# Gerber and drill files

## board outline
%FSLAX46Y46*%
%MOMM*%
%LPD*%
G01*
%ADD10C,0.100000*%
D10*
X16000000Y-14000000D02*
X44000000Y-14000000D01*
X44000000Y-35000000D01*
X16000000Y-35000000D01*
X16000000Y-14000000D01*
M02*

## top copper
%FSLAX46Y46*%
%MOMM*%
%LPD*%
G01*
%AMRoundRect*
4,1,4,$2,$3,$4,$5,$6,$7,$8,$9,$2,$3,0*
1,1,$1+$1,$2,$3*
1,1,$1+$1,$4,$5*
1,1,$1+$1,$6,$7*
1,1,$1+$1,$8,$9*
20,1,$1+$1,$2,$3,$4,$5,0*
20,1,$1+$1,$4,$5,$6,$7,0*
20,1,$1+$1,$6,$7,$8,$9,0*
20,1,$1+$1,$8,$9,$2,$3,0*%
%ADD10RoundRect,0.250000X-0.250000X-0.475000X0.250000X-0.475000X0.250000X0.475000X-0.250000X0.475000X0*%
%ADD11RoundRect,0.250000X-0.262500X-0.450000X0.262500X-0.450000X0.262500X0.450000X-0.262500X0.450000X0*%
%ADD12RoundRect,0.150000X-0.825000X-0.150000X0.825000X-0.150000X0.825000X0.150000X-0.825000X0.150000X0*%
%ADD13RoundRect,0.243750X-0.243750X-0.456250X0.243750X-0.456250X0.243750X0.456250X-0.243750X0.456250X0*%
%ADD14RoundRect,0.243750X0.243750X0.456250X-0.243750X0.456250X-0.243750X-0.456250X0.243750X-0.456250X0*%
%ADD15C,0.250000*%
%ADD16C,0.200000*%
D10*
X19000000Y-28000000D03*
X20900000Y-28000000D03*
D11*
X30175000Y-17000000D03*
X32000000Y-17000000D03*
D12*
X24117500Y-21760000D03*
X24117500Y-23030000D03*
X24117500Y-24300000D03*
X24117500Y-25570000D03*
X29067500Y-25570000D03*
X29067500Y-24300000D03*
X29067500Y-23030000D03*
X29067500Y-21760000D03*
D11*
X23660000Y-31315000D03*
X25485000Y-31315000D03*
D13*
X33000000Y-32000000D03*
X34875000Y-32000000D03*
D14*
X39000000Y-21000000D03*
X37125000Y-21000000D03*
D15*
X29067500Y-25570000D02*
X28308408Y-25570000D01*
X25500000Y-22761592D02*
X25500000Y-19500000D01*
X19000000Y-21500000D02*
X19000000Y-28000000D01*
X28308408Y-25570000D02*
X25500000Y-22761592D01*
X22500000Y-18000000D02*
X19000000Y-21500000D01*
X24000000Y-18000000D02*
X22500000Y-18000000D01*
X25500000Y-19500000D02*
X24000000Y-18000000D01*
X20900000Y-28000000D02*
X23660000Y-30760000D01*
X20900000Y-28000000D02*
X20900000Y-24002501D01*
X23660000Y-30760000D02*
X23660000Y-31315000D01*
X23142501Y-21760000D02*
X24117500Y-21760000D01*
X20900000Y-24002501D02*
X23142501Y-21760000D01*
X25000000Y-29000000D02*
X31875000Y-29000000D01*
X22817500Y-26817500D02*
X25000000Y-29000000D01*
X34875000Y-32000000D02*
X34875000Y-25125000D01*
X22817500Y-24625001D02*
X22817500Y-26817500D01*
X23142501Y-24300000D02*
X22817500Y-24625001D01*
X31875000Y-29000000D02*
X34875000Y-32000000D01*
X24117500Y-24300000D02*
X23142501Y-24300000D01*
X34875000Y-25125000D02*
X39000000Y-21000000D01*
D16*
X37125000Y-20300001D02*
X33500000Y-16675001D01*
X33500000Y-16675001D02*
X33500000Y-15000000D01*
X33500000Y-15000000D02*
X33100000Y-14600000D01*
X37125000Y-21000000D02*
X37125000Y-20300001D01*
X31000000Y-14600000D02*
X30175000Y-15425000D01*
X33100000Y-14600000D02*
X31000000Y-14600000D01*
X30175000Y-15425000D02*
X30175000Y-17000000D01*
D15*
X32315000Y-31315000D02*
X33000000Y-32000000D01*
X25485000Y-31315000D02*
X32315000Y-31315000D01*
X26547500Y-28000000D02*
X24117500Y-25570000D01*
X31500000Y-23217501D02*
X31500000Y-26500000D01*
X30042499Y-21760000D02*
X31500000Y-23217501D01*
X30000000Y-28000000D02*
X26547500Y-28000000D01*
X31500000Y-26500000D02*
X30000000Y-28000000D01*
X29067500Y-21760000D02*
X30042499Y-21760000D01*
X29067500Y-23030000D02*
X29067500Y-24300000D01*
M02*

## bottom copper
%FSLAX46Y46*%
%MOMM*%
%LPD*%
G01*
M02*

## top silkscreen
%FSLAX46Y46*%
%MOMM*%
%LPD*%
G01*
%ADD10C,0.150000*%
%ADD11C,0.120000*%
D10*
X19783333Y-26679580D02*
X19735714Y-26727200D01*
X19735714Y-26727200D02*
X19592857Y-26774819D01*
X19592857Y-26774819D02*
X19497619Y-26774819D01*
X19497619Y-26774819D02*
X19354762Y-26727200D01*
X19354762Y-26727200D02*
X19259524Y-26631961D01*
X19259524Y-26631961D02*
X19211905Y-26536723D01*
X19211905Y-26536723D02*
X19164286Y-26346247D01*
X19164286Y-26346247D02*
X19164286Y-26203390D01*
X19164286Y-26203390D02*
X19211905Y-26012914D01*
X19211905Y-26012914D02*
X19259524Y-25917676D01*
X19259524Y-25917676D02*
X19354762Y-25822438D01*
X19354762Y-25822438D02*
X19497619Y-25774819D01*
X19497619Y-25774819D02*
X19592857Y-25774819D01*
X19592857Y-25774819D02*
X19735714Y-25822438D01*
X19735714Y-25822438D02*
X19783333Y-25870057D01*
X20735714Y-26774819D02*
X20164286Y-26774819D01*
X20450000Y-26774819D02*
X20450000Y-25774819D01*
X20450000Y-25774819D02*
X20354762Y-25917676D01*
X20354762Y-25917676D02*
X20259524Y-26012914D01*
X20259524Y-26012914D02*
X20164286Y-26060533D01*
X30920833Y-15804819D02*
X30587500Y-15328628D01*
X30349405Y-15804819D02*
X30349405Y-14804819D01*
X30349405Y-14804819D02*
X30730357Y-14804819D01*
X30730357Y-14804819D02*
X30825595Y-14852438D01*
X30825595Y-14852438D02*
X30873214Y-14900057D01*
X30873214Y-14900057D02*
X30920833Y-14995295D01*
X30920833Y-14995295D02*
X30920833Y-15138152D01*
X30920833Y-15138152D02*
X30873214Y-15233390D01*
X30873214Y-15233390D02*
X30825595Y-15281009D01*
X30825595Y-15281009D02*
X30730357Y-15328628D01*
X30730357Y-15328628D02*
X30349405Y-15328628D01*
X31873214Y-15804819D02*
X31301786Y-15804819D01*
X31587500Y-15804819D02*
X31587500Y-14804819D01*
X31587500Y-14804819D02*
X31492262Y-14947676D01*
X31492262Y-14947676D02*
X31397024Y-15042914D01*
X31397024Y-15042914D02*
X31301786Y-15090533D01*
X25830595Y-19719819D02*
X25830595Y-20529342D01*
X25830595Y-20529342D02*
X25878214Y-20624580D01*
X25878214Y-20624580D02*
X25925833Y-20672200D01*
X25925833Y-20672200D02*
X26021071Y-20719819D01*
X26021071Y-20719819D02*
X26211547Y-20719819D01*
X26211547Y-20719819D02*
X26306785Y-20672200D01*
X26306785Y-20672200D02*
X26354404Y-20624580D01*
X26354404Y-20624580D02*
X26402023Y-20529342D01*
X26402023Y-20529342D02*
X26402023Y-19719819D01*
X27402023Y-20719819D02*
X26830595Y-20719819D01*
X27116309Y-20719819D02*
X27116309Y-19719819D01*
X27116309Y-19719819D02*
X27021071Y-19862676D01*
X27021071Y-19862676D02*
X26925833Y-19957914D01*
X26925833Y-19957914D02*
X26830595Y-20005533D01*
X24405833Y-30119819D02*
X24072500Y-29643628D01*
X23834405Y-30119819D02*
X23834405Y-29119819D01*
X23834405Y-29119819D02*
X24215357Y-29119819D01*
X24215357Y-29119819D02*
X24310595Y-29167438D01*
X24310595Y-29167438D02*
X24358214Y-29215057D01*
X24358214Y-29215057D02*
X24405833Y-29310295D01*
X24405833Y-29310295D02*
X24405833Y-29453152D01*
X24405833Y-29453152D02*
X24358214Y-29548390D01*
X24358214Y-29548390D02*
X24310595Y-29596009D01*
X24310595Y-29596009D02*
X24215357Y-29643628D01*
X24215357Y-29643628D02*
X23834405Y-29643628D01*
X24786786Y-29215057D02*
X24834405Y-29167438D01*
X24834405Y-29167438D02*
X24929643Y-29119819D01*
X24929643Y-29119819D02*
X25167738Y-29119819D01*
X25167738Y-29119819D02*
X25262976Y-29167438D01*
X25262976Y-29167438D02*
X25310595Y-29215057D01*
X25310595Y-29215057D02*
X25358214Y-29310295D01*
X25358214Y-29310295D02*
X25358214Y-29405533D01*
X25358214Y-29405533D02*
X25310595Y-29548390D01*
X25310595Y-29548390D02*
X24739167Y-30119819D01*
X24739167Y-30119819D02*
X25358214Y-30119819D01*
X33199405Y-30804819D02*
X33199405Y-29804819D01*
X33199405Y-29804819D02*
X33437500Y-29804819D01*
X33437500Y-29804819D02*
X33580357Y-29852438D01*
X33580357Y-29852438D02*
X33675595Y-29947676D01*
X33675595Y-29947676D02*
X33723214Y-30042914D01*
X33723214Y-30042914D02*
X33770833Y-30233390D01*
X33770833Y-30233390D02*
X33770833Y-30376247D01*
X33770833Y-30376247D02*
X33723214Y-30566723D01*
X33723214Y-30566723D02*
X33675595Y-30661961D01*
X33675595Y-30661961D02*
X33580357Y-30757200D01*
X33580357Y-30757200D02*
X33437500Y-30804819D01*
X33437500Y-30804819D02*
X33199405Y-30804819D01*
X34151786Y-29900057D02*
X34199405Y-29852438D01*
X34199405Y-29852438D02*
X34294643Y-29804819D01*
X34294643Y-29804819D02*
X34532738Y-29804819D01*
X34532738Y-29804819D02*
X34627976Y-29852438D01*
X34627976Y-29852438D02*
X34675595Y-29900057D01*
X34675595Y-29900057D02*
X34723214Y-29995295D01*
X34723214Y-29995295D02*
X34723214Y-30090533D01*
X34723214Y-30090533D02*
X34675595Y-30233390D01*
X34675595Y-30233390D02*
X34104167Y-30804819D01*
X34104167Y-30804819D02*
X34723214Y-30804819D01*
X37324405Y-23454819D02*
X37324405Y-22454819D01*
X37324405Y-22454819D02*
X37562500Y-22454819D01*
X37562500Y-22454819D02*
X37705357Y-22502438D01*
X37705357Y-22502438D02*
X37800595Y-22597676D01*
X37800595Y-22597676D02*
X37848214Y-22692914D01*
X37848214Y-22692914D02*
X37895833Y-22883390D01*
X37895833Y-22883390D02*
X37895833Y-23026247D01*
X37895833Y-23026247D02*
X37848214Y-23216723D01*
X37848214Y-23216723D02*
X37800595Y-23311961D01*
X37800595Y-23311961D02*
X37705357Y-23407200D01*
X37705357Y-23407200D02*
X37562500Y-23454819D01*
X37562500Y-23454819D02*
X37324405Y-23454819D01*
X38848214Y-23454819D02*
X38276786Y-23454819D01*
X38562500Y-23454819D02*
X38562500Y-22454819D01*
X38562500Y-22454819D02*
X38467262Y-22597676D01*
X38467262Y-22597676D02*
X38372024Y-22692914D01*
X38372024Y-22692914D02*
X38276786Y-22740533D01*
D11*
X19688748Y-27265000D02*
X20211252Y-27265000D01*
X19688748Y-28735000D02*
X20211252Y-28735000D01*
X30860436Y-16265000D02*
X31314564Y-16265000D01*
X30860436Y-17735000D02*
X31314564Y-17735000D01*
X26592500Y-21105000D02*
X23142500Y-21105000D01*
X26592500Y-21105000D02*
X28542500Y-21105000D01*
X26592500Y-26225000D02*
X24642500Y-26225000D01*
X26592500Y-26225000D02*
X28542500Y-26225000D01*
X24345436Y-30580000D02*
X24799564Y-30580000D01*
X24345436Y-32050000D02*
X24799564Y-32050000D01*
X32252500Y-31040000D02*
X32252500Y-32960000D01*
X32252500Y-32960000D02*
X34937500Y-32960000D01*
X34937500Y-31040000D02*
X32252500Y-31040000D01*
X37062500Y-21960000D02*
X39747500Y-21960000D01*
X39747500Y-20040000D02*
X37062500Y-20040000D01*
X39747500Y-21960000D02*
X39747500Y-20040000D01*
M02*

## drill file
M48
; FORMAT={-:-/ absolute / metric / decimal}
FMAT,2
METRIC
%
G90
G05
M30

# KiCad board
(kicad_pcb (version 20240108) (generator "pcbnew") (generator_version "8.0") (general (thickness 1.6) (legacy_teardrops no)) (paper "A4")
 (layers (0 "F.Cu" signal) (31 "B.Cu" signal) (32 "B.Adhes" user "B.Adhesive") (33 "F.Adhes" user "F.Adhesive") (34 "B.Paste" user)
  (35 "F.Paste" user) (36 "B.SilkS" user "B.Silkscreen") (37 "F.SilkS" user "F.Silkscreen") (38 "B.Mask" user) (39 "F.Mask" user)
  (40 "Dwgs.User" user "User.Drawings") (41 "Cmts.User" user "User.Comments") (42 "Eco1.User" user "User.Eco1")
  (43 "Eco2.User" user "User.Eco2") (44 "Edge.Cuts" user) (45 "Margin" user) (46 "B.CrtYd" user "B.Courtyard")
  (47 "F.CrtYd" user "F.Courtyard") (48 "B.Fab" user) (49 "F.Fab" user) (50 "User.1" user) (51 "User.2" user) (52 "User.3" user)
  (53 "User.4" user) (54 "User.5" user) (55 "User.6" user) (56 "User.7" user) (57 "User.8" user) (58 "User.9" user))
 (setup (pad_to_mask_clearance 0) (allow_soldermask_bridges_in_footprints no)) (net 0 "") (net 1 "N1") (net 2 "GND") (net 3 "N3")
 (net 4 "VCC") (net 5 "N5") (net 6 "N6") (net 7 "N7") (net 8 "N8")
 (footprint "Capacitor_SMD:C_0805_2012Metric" (layer "F.Cu") (at 19.95 28)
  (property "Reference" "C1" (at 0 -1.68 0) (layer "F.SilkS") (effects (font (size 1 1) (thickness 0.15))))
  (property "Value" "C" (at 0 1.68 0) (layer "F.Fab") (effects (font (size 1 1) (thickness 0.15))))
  (fp_line (start -0.261252 -0.735) (end 0.261252 -0.735) (stroke (width 0.12) (type solid)) (layer "F.SilkS"))
  (fp_line (start -0.261252 0.735) (end 0.261252 0.735) (stroke (width 0.12) (type solid)) (layer "F.SilkS"))
  (pad "1" smd roundrect (at -0.95 0) (size 1 1.45) (layers "F.Cu" "F.Paste" "F.Mask") (roundrect_rratio 0.25) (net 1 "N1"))
  (pad "2" smd roundrect (at 0.95 0) (size 1 1.45) (layers "F.Cu" "F.Paste" "F.Mask") (roundrect_rratio 0.25) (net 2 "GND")))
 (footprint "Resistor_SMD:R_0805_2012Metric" (layer "F.Cu") (at 31.0875 17)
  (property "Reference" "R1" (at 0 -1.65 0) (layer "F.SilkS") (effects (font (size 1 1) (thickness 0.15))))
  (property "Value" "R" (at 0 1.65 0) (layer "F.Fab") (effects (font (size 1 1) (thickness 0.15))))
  (fp_line (start -0.227064 -0.735) (end 0.227064 -0.735) (stroke (width 0.12) (type solid)) (layer "F.SilkS"))
  (fp_line (start -0.227064 0.735) (end 0.227064 0.735) (stroke (width 0.12) (type solid)) (layer "F.SilkS"))
  (pad "1" smd roundrect (at -0.9125 0) (size 1.025 1.4) (layers "F.Cu" "F.Paste" "F.Mask") (roundrect_rratio 0.243902) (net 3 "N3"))
  (pad "2" smd roundrect (at 0.9125 0) (size 1.025 1.4) (layers "F.Cu" "F.Paste" "F.Mask") (roundrect_rratio 0.243902) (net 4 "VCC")))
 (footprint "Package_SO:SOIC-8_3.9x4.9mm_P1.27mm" (layer "F.Cu") (at 26.5925 23.665)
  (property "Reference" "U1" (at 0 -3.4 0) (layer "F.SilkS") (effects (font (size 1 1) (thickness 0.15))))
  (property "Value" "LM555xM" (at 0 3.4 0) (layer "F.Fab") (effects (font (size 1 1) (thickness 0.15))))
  (fp_line (start 0 -2.56) (end -3.45 -2.56) (stroke (width 0.12) (type solid)) (layer "F.SilkS"))
  (fp_line (start 0 -2.56) (end 1.95 -2.56) (stroke (width 0.12) (type solid)) (layer "F.SilkS"))
  (fp_line (start 0 2.56) (end -1.95 2.56) (stroke (width 0.12) (type solid)) (layer "F.SilkS"))
  (fp_line (start 0 2.56) (end 1.95 2.56) (stroke (width 0.12) (type solid)) (layer "F.SilkS"))
  (pad "1" smd roundrect (at -2.475 -1.905) (size 1.95 0.6) (layers "F.Cu" "F.Paste" "F.Mask") (roundrect_rratio 0.25) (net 2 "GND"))
  (pad "2" smd roundrect (at -2.475 -0.635) (size 1.95 0.6) (layers "F.Cu" "F.Paste" "F.Mask") (roundrect_rratio 0.25) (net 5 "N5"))
  (pad "3" smd roundrect (at -2.475 0.635) (size 1.95 0.6) (layers "F.Cu" "F.Paste" "F.Mask") (roundrect_rratio 0.25) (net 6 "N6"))
  (pad "4" smd roundrect (at -2.475 1.905) (size 1.95 0.6) (layers "F.Cu" "F.Paste" "F.Mask") (roundrect_rratio 0.25) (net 4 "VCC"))
  (pad "5" smd roundrect (at 2.475 1.905) (size 1.95 0.6) (layers "F.Cu" "F.Paste" "F.Mask") (roundrect_rratio 0.25) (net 1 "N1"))
  (pad "6" smd roundrect (at 2.475 0.635) (size 1.95 0.6) (layers "F.Cu" "F.Paste" "F.Mask") (roundrect_rratio 0.25) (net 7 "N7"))
  (pad "7" smd roundrect (at 2.475 -0.635) (size 1.95 0.6) (layers "F.Cu" "F.Paste" "F.Mask") (roundrect_rratio 0.25) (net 7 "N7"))
  (pad "8" smd roundrect (at 2.475 -1.905) (size 1.95 0.6) (layers "F.Cu" "F.Paste" "F.Mask") (roundrect_rratio 0.25) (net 4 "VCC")))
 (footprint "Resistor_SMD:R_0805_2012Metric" (layer "F.Cu") (at 24.5725 31.315)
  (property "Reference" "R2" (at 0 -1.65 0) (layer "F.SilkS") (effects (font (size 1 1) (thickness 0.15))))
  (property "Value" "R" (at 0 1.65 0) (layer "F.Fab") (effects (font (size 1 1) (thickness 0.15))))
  (fp_line (start -0.227064 -0.735) (end 0.227064 -0.735) (stroke (width 0.12) (type solid)) (layer "F.SilkS"))
  (fp_line (start -0.227064 0.735) (end 0.227064 0.735) (stroke (width 0.12) (type solid)) (layer "F.SilkS"))
  (pad "1" smd roundrect (at -0.9125 0) (size 1.025 1.4) (layers "F.Cu" "F.Paste" "F.Mask") (roundrect_rratio 0.243902) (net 2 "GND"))
  (pad "2" smd roundrect (at 0.9125 0) (size 1.025 1.4) (layers "F.Cu" "F.Paste" "F.Mask") (roundrect_rratio 0.243902) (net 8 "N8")))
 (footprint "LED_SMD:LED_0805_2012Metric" (layer "F.Cu") (at 33.9375 32)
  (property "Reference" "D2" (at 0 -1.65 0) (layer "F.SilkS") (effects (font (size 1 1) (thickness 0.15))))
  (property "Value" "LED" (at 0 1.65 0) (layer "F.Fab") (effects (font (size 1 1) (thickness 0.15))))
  (fp_line (start -1.685 -0.96) (end -1.685 0.96) (stroke (width 0.12) (type solid)) (layer "F.SilkS"))
  (fp_line (start -1.685 0.96) (end 1 0.96) (stroke (width 0.12) (type solid)) (layer "F.SilkS"))
  (fp_line (start 1 -0.96) (end -1.685 -0.96) (stroke (width 0.12) (type solid)) (layer "F.SilkS"))
  (pad "1" smd roundrect (at -0.9375 0) (size 0.975 1.4) (layers "F.Cu" "F.Paste" "F.Mask") (roundrect_rratio 0.25) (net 8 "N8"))
  (pad "2" smd roundrect (at 0.9375 0) (size 0.975 1.4) (layers "F.Cu" "F.Paste" "F.Mask") (roundrect_rratio 0.25) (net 6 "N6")))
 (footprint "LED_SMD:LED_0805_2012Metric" (layer "F.Cu") (at 38.0625 21 180)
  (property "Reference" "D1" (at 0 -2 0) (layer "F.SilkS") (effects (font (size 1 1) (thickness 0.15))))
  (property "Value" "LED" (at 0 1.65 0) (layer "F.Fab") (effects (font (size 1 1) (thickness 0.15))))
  (fp_line (start 1 -0.96) (end -1.685 -0.96) (stroke (width 0.12) (type solid)) (layer "F.SilkS"))
  (fp_line (start -1.685 0.96) (end 1 0.96) (stroke (width 0.12) (type solid)) (layer "F.SilkS"))
  (fp_line (start -1.685 -0.96) (end -1.685 0.96) (stroke (width 0.12) (type solid)) (layer "F.SilkS"))
  (pad "1" smd roundrect (at -0.9375 0 180) (size 0.975 1.4) (layers "F.Cu" "F.Paste" "F.Mask") (roundrect_rratio 0.25) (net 6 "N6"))
  (pad "2" smd roundrect (at 0.9375 0 180) (size 0.975 1.4) (layers "F.Cu" "F.Paste" "F.Mask") (roundrect_rratio 0.25) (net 3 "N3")))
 (gr_rect (start 16 14) (end 44 35) (stroke (width 0.1) (type default)) (fill none) (layer "Edge.Cuts"))
 (segment (start 29.0675 25.57) (end 28.308408 25.57) (width 0.25) (layer "F.Cu") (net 1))
 (segment (start 25.5 22.761592) (end 25.5 19.5) (width 0.25) (layer "F.Cu") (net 1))
 (segment (start 19 21.5) (end 19 28) (width 0.25) (layer "F.Cu") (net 1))
 (segment (start 28.308408 25.57) (end 25.5 22.761592) (width 0.25) (layer "F.Cu") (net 1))
 (segment (start 22.5 18) (end 19 21.5) (width 0.25) (layer "F.Cu") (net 1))
 (segment (start 24 18) (end 22.5 18) (width 0.25) (layer "F.Cu") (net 1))
 (segment (start 25.5 19.5) (end 24 18) (width 0.25) (layer "F.Cu") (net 1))
 (segment (start 20.9 28) (end 23.66 30.76) (width 0.25) (layer "F.Cu") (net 2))
 (segment (start 20.9 28) (end 20.9 24.002501) (width 0.25) (layer "F.Cu") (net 2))
 (segment (start 23.66 30.76) (end 23.66 31.315) (width 0.25) (layer "F.Cu") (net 2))
 (segment (start 23.142501 21.76) (end 24.1175 21.76) (width 0.25) (layer "F.Cu") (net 2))
 (segment (start 20.9 24.002501) (end 23.142501 21.76) (width 0.25) (layer "F.Cu") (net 2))
 (segment (start 25 29) (end 31.875 29) (width 0.25) (layer "F.Cu") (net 6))
 (segment (start 22.8175 26.8175) (end 25 29) (width 0.25) (layer "F.Cu") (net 6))
 (segment (start 34.875 32) (end 34.875 25.125) (width 0.25) (layer "F.Cu") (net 6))
 (segment (start 22.8175 24.625001) (end 22.8175 26.8175) (width 0.25) (layer "F.Cu") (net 6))
 (segment (start 23.142501 24.3) (end 22.8175 24.625001) (width 0.25) (layer "F.Cu") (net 6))
 (segment (start 31.875 29) (end 34.875 32) (width 0.25) (layer "F.Cu") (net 6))
 (segment (start 24.1175 24.3) (end 23.142501 24.3) (width 0.25) (layer "F.Cu") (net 6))
 (segment (start 34.875 25.125) (end 39 21) (width 0.25) (layer "F.Cu") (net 6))
 (segment (start 37.125 20.300001) (end 33.5 16.675001) (width 0.2) (layer "F.Cu") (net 3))
 (segment (start 33.5 16.675001) (end 33.5 15) (width 0.2) (layer "F.Cu") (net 3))
 (segment (start 33.5 15) (end 33.1 14.6) (width 0.2) (layer "F.Cu") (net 3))
 (segment (start 37.125 21) (end 37.125 20.300001) (width 0.2) (layer "F.Cu") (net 3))
 (segment (start 31 14.6) (end 30.175 15.425) (width 0.2) (layer "F.Cu") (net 3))
 (segment (start 33.1 14.6) (end 31 14.6) (width 0.2) (layer "F.Cu") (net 3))
 (segment (start 30.175 15.425) (end 30.175 17) (width 0.2) (layer "F.Cu") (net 3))
 (segment (start 32.315 31.315) (end 33 32) (width 0.25) (layer "F.Cu") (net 8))
 (segment (start 25.485 31.315) (end 32.315 31.315) (width 0.25) (layer "F.Cu") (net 8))
 (segment (start 26.5475 28) (end 24.1175 25.57) (width 0.25) (layer "F.Cu") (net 4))
 (segment (start 31.5 23.217501) (end 31.5 26.5) (width 0.25) (layer "F.Cu") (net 4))
 (segment (start 30.042499 21.76) (end 31.5 23.217501) (width 0.25) (layer "F.Cu") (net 4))
 (segment (start 30 28) (end 26.5475 28) (width 0.25) (layer "F.Cu") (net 4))
 (segment (start 31.5 26.5) (end 30 28) (width 0.25) (layer "F.Cu") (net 4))
 (segment (start 29.0675 21.76) (end 30.042499 21.76) (width 0.25) (layer "F.Cu") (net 4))
 (segment (start 29.0675 23.03) (end 29.0675 24.3) (width 0.25) (layer "F.Cu") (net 7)))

